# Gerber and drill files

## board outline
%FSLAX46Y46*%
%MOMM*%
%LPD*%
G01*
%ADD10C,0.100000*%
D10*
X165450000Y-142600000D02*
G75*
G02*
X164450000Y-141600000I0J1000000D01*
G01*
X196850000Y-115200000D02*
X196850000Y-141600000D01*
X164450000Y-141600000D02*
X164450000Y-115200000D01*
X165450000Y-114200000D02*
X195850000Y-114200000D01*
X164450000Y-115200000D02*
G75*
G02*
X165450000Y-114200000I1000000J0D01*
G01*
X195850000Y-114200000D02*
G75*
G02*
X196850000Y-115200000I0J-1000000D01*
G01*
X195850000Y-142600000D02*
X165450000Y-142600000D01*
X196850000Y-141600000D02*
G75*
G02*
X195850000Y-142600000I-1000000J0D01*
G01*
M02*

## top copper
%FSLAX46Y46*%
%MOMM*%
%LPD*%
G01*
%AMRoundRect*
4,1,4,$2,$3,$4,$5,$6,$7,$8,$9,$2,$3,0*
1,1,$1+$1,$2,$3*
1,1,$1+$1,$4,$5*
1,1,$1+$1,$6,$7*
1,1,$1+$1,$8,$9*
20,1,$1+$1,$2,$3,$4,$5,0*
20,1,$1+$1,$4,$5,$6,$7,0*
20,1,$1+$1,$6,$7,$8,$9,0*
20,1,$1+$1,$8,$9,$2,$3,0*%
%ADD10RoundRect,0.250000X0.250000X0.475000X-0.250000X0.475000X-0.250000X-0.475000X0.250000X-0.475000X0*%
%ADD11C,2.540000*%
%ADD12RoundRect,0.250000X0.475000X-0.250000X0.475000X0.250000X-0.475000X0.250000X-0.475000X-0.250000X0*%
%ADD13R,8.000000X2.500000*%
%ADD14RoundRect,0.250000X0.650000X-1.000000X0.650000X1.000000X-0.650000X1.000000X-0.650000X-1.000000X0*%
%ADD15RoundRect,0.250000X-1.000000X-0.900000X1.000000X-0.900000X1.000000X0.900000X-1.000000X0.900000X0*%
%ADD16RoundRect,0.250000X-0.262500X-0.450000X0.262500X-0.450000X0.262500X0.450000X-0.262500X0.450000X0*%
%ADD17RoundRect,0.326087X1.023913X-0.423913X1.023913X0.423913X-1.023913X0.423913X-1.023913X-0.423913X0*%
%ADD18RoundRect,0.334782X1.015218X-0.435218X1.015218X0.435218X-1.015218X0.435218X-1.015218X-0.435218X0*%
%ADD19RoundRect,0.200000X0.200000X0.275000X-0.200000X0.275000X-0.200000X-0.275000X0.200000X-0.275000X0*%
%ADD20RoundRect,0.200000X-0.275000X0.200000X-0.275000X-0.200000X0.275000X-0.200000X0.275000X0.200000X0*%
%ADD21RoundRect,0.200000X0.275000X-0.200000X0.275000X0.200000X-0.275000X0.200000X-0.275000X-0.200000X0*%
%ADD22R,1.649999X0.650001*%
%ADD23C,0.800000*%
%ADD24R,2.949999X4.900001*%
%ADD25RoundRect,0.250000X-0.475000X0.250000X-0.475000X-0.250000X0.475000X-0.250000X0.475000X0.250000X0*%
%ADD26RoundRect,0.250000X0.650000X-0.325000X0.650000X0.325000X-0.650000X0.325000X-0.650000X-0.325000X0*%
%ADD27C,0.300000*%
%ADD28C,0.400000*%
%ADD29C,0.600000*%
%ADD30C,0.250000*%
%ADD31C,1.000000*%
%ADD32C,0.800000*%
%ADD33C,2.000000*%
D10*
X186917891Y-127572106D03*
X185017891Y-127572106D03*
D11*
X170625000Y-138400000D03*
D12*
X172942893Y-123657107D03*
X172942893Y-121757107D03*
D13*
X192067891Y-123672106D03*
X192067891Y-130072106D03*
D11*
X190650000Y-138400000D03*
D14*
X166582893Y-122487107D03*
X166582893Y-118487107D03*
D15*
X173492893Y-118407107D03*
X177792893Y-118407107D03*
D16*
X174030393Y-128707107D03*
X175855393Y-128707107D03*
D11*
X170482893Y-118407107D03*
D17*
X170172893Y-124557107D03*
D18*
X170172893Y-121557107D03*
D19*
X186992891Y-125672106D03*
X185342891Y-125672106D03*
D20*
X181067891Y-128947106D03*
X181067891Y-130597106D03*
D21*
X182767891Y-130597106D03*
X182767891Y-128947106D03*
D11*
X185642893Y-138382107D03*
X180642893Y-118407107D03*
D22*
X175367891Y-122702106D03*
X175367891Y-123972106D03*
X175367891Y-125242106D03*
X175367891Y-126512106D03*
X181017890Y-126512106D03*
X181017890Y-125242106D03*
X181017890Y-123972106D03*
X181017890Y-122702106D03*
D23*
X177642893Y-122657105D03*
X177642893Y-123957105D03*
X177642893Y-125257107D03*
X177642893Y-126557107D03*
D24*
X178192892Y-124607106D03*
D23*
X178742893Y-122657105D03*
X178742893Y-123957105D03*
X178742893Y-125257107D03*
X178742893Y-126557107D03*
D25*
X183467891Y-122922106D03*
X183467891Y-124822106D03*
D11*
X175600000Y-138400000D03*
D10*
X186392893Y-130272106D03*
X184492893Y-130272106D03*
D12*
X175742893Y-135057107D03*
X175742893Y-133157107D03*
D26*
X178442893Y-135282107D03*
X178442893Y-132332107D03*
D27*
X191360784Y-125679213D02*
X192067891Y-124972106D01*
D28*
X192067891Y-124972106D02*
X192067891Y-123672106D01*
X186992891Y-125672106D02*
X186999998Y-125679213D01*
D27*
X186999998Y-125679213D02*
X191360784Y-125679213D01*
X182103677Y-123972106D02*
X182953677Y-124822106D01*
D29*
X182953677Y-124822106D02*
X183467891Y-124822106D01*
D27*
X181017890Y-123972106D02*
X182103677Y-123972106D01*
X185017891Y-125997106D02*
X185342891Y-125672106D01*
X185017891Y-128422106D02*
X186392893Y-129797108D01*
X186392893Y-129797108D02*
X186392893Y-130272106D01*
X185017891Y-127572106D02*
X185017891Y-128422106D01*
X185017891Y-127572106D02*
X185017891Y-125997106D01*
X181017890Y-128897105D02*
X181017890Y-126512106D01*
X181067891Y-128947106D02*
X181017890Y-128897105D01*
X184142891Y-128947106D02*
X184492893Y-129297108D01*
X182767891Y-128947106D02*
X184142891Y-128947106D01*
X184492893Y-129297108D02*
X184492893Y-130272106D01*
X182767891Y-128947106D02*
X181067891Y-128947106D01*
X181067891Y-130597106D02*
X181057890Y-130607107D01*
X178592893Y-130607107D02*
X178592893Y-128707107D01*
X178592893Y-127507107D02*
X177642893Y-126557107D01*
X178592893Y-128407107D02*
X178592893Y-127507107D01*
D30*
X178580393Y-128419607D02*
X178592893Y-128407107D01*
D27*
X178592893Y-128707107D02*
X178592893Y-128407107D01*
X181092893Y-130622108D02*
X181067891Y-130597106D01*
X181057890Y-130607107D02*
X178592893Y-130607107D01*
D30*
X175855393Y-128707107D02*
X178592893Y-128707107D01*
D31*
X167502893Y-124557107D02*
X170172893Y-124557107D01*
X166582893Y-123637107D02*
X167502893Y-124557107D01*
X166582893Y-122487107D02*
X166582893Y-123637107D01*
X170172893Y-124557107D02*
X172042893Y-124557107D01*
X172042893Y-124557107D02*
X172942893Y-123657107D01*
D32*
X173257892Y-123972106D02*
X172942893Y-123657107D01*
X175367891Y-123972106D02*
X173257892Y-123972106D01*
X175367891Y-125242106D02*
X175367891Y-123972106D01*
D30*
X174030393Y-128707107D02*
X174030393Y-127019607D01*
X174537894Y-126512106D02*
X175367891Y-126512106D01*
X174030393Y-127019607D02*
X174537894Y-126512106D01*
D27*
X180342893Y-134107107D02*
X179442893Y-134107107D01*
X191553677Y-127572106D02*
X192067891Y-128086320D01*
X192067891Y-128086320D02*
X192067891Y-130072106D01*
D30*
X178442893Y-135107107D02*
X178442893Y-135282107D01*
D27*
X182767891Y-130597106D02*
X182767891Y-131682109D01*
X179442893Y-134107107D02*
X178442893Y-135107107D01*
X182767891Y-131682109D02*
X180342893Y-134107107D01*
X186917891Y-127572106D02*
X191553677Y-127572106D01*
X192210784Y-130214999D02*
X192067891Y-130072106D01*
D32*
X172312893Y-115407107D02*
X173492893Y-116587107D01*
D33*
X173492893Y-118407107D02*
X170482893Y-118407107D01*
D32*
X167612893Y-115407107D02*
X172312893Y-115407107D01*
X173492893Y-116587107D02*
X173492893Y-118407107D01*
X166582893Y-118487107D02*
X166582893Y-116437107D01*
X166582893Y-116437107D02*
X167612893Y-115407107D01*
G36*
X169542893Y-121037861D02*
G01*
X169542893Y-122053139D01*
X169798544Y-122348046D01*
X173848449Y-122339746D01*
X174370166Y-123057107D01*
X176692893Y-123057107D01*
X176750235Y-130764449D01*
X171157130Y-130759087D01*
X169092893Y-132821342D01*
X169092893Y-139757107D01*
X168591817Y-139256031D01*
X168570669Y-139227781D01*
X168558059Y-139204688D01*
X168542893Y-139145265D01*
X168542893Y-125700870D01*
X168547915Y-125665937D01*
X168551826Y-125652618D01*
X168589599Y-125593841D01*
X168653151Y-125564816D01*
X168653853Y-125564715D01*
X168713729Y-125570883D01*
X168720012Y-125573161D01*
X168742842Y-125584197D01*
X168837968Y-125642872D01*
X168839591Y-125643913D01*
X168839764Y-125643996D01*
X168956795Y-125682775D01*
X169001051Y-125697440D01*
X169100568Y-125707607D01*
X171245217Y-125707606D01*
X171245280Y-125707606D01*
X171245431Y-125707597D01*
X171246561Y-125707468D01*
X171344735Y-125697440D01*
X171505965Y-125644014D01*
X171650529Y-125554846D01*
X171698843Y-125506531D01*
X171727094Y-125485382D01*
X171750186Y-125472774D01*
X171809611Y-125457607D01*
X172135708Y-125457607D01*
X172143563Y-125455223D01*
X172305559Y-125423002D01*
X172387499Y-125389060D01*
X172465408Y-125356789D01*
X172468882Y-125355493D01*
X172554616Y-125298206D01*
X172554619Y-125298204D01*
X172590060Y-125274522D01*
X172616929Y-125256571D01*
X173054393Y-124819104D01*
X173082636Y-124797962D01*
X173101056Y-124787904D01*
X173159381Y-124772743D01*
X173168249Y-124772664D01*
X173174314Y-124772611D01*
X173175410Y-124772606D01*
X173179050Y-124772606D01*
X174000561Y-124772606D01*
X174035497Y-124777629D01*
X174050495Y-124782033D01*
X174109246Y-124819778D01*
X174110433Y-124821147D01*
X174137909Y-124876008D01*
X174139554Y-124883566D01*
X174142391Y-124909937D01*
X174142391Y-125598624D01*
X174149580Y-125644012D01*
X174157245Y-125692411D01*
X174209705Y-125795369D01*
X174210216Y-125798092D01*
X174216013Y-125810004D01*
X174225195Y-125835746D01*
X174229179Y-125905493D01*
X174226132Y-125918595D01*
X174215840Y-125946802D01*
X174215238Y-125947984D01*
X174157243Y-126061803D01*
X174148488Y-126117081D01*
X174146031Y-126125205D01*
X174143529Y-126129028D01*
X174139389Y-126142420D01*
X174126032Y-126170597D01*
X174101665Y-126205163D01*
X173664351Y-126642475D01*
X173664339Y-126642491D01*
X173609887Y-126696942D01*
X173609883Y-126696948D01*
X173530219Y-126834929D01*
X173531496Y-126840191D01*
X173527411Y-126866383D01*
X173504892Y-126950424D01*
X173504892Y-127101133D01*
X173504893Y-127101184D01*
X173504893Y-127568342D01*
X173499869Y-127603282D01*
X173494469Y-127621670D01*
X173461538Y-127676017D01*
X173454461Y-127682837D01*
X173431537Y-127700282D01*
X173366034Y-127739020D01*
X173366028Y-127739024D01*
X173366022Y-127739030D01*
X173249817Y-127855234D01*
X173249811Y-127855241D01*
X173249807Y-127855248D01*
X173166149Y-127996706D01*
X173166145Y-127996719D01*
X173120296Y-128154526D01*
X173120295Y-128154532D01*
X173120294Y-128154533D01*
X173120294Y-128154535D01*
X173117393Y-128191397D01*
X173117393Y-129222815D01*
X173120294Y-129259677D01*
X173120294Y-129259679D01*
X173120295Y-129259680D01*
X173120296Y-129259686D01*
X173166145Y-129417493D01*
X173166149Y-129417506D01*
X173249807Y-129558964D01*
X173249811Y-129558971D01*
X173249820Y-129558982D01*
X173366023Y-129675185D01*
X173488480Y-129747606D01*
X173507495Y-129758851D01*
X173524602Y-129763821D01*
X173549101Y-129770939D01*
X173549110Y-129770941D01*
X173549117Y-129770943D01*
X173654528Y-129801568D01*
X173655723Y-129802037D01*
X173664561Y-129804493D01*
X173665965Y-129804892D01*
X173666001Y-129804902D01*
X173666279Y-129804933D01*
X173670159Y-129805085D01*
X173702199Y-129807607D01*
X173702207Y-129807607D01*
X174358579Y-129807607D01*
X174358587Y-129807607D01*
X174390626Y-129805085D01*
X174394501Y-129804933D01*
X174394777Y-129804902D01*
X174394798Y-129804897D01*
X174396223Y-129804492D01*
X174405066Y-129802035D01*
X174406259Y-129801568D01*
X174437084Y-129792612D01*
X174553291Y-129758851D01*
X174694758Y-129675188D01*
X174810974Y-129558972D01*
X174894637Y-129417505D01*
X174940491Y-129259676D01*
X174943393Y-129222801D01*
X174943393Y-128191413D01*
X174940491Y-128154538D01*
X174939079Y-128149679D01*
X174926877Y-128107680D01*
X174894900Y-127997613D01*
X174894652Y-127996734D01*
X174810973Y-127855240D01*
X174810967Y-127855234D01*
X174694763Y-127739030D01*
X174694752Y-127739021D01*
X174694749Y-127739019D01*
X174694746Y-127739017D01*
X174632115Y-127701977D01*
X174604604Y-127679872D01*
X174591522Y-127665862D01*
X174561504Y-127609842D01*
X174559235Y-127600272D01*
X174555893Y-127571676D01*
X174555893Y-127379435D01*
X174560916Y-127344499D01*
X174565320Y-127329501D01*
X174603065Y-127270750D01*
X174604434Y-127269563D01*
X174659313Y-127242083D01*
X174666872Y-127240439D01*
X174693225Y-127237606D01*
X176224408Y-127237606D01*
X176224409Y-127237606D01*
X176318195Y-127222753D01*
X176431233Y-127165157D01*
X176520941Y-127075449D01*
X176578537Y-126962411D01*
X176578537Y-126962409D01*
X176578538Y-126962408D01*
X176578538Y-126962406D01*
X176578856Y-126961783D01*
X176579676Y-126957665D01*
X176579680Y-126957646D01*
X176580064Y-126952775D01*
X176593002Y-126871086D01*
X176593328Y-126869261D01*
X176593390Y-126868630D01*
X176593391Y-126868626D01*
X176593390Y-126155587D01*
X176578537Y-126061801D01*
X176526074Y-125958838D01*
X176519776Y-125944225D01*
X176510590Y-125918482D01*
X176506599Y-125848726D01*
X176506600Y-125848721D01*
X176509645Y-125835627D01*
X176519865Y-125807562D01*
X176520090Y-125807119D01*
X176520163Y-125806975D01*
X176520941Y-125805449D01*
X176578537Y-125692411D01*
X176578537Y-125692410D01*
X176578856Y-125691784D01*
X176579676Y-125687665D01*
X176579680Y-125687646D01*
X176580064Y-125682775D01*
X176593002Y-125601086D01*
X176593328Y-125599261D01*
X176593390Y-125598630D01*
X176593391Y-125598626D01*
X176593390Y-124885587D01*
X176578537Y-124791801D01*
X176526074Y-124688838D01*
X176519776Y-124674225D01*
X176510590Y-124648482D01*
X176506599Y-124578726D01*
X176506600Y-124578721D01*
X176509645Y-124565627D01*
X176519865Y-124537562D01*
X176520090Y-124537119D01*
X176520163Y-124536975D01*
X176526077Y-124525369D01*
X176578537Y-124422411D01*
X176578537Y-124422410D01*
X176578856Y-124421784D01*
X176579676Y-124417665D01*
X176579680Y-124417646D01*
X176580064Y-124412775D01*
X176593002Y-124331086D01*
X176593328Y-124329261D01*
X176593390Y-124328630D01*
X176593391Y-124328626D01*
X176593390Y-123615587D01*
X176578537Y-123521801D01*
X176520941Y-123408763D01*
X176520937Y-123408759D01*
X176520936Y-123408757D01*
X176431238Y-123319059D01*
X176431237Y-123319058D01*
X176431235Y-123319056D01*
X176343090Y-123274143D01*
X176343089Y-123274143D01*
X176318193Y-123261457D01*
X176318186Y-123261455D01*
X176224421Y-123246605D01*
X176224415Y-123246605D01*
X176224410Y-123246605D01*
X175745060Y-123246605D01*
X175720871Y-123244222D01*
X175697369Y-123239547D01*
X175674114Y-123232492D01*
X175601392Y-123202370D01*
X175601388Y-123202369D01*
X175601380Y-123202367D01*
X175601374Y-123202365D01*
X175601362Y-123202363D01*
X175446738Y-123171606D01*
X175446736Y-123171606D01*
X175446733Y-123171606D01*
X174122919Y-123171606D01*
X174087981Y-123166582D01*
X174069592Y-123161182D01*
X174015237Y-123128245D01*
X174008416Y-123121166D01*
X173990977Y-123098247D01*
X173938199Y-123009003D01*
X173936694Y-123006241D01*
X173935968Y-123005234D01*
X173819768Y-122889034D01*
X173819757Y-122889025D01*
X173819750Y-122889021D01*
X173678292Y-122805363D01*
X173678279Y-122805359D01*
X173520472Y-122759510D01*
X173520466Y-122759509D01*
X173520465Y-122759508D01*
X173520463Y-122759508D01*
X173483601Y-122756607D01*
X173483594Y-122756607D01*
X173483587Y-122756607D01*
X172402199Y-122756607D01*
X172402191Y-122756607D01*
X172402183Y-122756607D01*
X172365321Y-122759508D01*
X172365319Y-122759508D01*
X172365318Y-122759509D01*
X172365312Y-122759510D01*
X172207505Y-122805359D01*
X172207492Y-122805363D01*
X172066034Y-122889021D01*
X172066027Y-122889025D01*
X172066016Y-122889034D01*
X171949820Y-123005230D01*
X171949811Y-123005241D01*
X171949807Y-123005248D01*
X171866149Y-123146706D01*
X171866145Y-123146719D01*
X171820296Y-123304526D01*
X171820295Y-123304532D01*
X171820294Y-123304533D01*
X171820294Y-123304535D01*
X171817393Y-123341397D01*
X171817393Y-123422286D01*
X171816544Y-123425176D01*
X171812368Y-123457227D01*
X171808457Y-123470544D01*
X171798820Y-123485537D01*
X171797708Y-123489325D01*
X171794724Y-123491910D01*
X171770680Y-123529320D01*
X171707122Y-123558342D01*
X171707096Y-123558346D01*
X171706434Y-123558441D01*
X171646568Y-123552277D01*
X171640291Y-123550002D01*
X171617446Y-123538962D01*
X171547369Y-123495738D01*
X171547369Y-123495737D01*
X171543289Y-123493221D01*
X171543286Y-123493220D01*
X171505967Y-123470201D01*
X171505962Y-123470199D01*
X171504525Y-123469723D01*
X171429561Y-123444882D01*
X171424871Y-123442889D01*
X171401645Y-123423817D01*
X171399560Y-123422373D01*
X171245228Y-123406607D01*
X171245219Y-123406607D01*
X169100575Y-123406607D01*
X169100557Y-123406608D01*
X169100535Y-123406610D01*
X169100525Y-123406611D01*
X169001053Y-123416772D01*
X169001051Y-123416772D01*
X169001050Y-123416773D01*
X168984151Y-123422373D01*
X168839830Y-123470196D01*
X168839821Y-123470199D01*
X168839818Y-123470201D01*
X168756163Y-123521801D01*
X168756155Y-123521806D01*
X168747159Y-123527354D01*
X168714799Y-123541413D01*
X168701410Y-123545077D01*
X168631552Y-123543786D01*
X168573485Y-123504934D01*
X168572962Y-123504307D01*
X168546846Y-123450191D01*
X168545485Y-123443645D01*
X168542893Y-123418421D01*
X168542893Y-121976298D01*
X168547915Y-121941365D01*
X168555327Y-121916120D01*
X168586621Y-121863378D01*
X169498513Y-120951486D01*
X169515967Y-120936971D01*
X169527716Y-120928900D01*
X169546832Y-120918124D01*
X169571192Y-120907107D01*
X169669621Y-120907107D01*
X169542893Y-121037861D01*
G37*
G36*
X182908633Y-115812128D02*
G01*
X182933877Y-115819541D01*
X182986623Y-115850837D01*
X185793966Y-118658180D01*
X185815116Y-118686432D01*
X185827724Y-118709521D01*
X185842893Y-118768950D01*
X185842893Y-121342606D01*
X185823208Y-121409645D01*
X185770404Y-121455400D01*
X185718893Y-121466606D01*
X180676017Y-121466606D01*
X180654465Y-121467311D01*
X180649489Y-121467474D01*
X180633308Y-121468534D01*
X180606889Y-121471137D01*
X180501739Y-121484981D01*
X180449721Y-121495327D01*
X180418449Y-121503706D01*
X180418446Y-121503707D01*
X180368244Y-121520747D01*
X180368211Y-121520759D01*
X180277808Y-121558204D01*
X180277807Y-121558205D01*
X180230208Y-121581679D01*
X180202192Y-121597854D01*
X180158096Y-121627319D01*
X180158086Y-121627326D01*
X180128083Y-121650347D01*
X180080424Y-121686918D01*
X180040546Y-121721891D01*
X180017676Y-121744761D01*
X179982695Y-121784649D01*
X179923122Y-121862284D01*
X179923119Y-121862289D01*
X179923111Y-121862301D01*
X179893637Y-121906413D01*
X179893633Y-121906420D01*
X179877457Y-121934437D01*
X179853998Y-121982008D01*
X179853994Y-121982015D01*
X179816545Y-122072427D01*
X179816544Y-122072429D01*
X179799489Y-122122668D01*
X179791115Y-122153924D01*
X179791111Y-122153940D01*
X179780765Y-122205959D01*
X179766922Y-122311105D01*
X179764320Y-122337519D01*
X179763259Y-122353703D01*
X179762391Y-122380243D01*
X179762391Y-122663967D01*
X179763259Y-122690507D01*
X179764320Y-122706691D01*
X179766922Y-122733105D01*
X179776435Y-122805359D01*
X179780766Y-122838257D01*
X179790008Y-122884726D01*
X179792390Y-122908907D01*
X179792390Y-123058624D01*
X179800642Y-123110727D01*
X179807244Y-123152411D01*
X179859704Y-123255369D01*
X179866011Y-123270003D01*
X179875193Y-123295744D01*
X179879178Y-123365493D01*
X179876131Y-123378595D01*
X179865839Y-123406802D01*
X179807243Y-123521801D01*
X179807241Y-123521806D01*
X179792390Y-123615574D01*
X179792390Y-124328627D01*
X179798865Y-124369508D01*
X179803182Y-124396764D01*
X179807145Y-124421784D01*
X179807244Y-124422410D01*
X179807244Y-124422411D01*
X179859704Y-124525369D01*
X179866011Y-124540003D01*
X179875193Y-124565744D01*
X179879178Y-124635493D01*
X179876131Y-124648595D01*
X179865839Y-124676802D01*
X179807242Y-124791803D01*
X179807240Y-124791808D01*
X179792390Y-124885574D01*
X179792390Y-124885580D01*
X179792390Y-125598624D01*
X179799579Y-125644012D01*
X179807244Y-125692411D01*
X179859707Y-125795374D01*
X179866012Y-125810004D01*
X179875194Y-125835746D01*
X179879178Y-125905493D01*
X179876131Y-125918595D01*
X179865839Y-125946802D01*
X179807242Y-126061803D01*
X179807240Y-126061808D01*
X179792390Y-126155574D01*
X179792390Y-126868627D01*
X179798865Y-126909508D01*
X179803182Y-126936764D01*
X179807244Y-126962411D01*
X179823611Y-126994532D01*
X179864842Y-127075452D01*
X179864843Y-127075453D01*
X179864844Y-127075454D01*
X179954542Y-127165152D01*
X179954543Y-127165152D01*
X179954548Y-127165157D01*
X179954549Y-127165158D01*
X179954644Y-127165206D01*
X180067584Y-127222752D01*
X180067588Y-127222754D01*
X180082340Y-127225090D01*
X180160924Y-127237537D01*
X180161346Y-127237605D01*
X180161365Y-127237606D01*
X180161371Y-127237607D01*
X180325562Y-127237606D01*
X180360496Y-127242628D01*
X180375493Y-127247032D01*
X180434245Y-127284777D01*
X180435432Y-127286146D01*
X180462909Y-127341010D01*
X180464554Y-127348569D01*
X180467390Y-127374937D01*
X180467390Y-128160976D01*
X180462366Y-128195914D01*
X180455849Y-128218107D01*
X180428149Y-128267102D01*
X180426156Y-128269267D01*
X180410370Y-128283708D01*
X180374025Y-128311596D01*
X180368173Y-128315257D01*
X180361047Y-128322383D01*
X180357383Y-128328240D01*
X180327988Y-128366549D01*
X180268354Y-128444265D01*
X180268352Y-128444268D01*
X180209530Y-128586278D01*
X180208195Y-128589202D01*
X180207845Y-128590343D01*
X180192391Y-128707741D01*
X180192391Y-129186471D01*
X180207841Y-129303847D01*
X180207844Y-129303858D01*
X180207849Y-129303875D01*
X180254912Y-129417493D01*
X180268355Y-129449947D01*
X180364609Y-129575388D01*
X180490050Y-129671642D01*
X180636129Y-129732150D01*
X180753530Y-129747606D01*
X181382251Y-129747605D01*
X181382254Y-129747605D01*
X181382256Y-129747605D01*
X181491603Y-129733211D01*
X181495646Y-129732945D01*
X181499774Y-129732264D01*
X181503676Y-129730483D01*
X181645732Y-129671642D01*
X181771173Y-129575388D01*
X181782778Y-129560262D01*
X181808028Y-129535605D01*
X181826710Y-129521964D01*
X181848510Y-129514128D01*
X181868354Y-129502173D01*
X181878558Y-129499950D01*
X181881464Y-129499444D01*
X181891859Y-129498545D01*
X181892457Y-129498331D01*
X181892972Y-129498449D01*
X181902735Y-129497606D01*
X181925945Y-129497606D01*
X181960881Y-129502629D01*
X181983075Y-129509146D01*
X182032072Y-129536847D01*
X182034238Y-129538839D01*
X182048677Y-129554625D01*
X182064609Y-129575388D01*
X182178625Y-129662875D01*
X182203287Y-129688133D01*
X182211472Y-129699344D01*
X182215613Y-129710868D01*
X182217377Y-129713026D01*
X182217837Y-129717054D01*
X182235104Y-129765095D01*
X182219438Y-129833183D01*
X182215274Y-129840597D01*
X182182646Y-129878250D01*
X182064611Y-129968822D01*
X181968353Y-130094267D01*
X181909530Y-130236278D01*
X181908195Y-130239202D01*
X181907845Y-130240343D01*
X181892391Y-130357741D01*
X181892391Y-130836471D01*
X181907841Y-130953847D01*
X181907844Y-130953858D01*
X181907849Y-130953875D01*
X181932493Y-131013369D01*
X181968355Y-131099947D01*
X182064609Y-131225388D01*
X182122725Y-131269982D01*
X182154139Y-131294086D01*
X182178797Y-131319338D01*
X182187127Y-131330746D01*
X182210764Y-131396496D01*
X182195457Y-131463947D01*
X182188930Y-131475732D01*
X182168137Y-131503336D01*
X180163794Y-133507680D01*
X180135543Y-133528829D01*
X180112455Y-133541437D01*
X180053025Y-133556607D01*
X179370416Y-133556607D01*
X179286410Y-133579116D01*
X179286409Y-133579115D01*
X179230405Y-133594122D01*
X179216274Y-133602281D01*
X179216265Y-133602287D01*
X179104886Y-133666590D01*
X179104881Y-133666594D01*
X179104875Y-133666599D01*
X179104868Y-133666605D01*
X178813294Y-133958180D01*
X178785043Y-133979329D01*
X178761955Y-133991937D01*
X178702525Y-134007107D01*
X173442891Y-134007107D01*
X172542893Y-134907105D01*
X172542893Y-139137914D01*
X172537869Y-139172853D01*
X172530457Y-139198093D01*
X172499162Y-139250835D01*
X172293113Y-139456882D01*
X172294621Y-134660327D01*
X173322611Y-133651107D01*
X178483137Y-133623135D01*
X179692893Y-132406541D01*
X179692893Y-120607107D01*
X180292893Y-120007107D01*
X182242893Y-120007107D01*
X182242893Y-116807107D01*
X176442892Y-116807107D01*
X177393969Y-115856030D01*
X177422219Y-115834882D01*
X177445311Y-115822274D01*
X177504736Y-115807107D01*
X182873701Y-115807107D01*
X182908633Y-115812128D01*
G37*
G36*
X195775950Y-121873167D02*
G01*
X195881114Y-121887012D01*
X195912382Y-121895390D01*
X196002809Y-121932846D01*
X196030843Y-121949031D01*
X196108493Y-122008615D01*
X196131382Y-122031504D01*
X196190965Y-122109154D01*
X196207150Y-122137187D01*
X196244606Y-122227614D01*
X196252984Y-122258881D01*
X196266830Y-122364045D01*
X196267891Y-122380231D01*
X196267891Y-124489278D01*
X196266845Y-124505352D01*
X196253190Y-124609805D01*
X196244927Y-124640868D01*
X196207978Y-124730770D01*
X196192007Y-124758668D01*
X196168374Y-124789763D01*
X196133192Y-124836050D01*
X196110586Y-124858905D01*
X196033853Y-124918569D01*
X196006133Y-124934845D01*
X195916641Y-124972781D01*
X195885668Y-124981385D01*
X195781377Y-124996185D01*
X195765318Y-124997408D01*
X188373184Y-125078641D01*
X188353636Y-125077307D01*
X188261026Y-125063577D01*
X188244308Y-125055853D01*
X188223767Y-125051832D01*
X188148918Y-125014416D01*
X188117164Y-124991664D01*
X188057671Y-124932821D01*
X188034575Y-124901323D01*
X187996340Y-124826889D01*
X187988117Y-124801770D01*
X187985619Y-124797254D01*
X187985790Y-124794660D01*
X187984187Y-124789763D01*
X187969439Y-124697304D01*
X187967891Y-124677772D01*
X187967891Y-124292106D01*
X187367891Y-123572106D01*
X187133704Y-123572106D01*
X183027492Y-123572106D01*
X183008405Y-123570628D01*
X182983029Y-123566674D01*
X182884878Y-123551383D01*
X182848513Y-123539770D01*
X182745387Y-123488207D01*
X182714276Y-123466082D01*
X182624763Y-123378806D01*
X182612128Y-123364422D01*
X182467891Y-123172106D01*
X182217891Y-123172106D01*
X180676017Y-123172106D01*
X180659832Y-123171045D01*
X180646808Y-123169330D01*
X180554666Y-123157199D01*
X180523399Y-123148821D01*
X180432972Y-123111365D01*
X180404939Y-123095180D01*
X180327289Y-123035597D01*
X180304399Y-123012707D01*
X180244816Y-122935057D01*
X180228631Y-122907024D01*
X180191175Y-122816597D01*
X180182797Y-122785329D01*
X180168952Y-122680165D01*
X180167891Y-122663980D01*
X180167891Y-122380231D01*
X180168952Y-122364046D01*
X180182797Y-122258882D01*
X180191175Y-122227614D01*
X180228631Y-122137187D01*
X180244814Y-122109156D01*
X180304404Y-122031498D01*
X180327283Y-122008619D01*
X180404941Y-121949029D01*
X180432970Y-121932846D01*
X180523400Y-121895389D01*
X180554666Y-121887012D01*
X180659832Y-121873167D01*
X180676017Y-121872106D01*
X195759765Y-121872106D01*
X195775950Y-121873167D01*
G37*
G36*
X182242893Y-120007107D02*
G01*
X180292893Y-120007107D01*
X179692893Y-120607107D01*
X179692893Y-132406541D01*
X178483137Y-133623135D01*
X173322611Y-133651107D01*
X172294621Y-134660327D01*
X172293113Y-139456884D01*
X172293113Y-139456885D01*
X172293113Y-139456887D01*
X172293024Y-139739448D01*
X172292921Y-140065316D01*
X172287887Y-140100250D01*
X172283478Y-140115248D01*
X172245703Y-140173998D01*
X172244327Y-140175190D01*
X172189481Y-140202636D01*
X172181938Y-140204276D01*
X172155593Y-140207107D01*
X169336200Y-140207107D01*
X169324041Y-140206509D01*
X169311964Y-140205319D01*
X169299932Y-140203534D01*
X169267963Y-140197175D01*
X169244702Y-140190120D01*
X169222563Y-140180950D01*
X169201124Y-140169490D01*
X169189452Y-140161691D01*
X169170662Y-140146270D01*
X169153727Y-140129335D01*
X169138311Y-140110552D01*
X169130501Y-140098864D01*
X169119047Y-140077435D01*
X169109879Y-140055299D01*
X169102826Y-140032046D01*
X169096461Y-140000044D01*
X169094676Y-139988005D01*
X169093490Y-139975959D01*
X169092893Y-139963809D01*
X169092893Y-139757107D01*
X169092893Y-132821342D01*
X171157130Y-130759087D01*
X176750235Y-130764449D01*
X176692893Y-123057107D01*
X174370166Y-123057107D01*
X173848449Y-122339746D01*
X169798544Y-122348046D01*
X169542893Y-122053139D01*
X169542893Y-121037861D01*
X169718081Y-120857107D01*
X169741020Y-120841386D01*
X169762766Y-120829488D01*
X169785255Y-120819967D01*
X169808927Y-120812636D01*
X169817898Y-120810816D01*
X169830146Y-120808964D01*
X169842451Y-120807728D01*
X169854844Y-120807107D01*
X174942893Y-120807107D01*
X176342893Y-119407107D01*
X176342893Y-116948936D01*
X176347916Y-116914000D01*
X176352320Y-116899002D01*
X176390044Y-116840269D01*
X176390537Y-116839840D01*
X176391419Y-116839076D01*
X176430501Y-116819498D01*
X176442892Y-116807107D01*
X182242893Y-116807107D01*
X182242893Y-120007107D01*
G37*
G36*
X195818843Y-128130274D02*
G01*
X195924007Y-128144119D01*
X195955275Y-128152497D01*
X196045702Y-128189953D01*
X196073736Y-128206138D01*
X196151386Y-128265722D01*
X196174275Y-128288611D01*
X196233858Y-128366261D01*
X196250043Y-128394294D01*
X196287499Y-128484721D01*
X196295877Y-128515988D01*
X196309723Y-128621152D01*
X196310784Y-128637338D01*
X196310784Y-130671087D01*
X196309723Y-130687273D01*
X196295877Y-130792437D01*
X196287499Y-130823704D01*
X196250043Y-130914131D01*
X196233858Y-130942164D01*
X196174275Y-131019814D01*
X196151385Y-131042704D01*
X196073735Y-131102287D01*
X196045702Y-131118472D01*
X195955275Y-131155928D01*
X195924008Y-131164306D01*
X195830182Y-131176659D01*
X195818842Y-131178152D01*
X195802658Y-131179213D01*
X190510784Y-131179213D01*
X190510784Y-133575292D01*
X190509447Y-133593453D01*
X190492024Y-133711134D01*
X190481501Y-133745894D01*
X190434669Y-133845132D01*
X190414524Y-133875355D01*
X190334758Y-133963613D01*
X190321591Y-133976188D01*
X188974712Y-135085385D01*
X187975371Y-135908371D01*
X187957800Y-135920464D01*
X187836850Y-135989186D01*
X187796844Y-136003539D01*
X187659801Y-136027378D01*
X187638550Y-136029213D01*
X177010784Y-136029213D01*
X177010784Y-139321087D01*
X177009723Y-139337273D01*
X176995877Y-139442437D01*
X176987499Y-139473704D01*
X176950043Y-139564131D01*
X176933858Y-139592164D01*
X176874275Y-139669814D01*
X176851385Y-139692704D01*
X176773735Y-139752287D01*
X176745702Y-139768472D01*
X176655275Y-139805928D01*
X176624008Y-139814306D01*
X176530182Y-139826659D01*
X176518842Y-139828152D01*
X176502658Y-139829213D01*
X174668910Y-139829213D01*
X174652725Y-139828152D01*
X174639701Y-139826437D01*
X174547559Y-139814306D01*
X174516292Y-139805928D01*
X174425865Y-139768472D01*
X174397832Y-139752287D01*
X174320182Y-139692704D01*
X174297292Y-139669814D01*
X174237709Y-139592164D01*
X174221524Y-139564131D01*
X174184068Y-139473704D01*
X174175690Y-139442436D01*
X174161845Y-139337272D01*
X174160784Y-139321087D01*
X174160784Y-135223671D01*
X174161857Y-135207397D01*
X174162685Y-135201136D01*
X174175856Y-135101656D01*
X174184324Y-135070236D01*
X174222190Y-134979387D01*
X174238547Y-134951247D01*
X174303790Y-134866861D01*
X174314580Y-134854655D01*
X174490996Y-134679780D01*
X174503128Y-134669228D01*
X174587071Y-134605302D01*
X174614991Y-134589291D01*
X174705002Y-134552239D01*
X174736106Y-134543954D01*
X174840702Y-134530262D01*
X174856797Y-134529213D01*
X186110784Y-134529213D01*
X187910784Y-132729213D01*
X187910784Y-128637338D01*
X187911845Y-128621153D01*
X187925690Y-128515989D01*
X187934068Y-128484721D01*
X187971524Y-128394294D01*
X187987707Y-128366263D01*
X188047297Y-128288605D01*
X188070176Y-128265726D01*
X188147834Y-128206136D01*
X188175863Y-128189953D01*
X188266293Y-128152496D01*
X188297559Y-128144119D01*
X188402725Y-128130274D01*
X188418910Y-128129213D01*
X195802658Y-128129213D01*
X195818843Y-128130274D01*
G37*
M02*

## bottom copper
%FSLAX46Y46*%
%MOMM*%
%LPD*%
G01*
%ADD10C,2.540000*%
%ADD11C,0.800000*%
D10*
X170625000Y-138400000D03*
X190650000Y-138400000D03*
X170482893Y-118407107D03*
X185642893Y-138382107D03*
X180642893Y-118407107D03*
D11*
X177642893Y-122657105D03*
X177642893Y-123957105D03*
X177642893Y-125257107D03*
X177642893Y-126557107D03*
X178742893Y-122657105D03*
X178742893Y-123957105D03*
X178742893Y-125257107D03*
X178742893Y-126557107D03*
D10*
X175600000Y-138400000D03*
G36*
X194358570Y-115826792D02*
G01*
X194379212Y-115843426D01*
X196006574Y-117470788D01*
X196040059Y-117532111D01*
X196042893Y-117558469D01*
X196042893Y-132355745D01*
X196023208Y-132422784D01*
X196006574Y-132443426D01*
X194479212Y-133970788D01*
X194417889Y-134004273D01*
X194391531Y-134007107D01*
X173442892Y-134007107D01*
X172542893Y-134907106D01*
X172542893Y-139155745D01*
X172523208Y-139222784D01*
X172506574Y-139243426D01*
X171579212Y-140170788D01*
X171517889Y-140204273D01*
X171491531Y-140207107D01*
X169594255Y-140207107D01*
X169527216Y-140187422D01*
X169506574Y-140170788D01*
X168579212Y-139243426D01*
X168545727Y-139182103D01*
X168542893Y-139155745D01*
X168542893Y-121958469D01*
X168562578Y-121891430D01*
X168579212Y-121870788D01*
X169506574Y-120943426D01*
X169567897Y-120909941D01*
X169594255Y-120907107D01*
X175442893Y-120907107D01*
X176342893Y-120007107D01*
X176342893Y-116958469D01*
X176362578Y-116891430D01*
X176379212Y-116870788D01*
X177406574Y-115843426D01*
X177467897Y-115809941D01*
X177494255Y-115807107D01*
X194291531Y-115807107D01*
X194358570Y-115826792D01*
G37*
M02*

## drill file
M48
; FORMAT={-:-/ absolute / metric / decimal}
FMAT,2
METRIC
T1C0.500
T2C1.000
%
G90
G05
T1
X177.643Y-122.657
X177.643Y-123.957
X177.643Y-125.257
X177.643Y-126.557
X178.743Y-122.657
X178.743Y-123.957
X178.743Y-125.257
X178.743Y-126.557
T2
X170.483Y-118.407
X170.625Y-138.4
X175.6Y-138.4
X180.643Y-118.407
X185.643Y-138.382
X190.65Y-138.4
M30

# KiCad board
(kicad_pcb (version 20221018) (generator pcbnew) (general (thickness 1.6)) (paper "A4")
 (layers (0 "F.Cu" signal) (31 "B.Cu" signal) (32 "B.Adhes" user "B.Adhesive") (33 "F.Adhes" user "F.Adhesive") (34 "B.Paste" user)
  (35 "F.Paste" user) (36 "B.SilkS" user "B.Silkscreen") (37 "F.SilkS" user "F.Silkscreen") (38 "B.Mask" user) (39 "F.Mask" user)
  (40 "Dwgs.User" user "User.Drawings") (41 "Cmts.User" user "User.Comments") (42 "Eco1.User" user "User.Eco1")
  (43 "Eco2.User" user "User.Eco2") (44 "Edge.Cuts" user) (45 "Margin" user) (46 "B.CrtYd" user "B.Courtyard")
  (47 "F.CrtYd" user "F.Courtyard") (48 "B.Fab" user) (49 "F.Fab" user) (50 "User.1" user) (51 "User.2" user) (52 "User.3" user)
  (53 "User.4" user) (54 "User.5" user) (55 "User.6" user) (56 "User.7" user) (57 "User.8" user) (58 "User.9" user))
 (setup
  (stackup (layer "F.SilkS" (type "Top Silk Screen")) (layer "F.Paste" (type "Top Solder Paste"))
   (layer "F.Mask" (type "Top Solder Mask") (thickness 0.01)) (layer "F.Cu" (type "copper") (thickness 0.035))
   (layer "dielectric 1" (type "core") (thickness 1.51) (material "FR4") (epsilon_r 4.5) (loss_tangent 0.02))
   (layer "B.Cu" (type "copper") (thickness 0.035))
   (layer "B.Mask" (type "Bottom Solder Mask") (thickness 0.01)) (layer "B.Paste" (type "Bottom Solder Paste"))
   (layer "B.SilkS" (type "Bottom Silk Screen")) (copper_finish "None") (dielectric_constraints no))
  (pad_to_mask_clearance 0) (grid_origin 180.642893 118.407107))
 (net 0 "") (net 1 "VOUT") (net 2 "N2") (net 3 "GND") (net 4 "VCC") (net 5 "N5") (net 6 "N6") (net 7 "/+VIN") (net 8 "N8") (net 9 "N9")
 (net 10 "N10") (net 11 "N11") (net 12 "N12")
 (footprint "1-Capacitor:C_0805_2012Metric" (layer "F.Cu") (at 185.967891 127.572106 180)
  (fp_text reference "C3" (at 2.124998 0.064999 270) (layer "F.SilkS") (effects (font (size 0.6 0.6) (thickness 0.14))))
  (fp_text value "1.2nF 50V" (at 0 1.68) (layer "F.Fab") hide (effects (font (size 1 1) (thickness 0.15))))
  (pad "1" smd roundrect (at -0.95 0 180) (size 1 1.45) (layers "F.Cu" "F.Paste" "F.Mask") (roundrect_rratio 0.25) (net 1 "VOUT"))
  (pad "2" smd roundrect (at 0.95 0 180) (size 1 1.45) (layers "F.Cu" "F.Paste" "F.Mask") (roundrect_rratio 0.25) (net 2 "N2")))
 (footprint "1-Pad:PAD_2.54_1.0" (layer "F.Cu") (at 170.625 138.4)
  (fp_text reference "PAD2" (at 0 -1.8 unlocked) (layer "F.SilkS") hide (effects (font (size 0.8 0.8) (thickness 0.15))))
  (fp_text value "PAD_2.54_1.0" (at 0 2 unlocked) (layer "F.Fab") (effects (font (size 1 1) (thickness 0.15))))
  (pad "1" thru_hole circle (at 0 0) (size 2.54 2.54) (drill 1) (layers "*.Cu" "*.Mask") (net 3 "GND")))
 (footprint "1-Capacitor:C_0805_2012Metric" (layer "F.Cu") (at 172.942893 122.707107 90)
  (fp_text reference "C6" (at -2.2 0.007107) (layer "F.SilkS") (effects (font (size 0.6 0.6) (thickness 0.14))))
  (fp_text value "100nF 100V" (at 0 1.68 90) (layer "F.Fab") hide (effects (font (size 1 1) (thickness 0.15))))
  (pad "1" smd roundrect (at -0.95 0 90) (size 1 1.45) (layers "F.Cu" "F.Paste" "F.Mask") (roundrect_rratio 0.25) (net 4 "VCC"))
  (pad "2" smd roundrect (at 0.95 0 90) (size 1 1.45) (layers "F.Cu" "F.Paste" "F.Mask") (roundrect_rratio 0.25) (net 3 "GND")))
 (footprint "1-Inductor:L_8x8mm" (layer "F.Cu") (at 192.067891 126.872106 -90)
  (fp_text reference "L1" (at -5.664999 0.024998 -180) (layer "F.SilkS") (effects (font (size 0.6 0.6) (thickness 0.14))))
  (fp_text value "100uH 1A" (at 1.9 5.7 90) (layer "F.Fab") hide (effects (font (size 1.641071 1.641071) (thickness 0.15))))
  (pad "1" smd rect (at -3.2 0) (size 8 2.5) (layers "F.Cu" "F.Paste" "F.Mask") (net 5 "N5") (solder_mask_margin 0.102))
  (pad "2" smd rect (at 3.2 0) (size 8 2.5) (layers "F.Cu" "F.Paste" "F.Mask") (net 1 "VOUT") (solder_mask_margin 0.102)))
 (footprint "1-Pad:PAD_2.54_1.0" (layer "F.Cu") (at 190.65 138.4)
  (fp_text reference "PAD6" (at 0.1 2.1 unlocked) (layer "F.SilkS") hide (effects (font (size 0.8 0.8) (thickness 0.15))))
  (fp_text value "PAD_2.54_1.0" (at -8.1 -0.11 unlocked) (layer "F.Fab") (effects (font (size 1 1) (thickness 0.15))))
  (pad "1" thru_hole circle (at 0 0) (size 2.54 2.54) (drill 1) (layers "*.Cu" "*.Mask") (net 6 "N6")))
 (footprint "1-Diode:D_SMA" (layer "F.Cu") (at 166.582893 120.487107 90)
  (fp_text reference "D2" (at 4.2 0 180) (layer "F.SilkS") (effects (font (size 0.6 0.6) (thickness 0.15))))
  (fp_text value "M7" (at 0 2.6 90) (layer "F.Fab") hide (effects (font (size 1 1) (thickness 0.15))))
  (pad "1" smd roundrect (at -2 0 90) (size 2.5 1.8) (layers "F.Cu" "F.Paste" "F.Mask") (roundrect_rratio 0.1388888889) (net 4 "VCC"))
  (pad "2" smd roundrect (at 2 0 90) (size 2.5 1.8) (layers "F.Cu" "F.Paste" "F.Mask") (roundrect_rratio 0.1388888889) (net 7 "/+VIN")))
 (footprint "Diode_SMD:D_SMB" (layer "F.Cu") (at 175.642893 118.407107)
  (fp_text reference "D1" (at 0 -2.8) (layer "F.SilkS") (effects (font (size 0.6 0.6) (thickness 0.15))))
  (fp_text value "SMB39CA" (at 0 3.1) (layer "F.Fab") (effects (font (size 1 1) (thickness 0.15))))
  (pad "1" smd roundrect (at -2.15 0) (size 2.5 2.3) (layers "F.Cu" "F.Paste" "F.Mask") (roundrect_rratio 0.1086956522) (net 7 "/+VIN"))
  (pad "2" smd roundrect (at 2.15 0) (size 2.5 2.3) (layers "F.Cu" "F.Paste" "F.Mask") (roundrect_rratio 0.1086956522) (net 3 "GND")))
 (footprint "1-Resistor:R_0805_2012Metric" (layer "F.Cu") (at 174.942893 128.707107)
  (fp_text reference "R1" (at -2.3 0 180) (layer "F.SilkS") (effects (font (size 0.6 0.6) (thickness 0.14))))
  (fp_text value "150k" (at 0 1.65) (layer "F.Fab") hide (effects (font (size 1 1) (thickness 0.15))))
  (pad "1" smd roundrect (at -0.9125 0) (size 1.025 1.4) (layers "F.Cu" "F.Paste" "F.Mask") (roundrect_rratio 0.243902439) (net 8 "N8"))
  (pad "2" smd roundrect (at 0.9125 0) (size 1.025 1.4) (layers "F.Cu" "F.Paste" "F.Mask") (roundrect_rratio 0.243902439) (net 3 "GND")))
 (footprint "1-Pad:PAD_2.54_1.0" (layer "F.Cu") (at 172.717893 118.332107)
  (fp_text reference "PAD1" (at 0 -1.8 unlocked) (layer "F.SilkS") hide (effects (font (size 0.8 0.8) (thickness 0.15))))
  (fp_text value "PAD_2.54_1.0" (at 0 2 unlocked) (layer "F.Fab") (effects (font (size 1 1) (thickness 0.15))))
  (pad "1" thru_hole circle (at -2.235 0.075) (size 2.54 2.54) (drill 1) (layers "*.Cu" "*.Mask") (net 7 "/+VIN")))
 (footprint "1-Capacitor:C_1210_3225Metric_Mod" (layer "F.Cu") (at 170.172893 123.057107 90)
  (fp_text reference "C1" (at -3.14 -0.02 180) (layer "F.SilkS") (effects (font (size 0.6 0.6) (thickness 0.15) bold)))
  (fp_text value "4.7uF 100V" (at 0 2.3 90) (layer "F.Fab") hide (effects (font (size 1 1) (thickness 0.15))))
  (pad "1" smd roundrect (at -1.5 0 90) (size 1.5 2.7) (layers "F.Cu" "F.Paste" "F.Mask") (roundrect_rratio 0.2173913333) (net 4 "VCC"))
  (pad "2" smd roundrect (at 1.5 0 90) (size 1.54 2.7) (layers "F.Cu" "F.Paste" "F.Mask") (roundrect_rratio 0.2173909091) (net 3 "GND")))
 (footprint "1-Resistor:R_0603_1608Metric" (layer "F.Cu") (at 186.167891 125.672106 180)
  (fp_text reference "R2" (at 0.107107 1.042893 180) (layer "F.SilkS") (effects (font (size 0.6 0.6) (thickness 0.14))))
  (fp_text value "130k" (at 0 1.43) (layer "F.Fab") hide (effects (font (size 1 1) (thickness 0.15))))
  (pad "1" smd roundrect (at -0.825 0 180) (size 0.8 0.95) (layers "F.Cu" "F.Paste" "F.Mask") (roundrect_rratio 0.25) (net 5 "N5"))
  (pad "2" smd roundrect (at 0.825 0 180) (size 0.8 0.95) (layers "F.Cu" "F.Paste" "F.Mask") (roundrect_rratio 0.25) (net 2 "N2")))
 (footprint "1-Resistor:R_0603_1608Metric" (layer "F.Cu") (at 181.067891 129.772106 -90)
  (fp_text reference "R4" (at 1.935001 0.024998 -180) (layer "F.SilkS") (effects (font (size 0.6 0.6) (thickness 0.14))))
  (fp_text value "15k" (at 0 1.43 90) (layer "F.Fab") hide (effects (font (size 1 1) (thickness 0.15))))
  (pad "1" smd roundrect (at -0.825 0 270) (size 0.8 0.95) (layers "F.Cu" "F.Paste" "F.Mask") (roundrect_rratio 0.25) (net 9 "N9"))
  (pad "2" smd roundrect (at 0.825 0 270) (size 0.8 0.95) (layers "F.Cu" "F.Paste" "F.Mask") (roundrect_rratio 0.25) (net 3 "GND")))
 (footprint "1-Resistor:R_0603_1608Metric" (layer "F.Cu") (at 182.767891 129.772106 90)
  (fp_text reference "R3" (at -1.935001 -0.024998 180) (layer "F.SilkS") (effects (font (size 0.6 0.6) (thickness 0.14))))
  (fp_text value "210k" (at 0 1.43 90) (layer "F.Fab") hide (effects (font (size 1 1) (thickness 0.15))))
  (pad "1" smd roundrect (at -0.825 0 90) (size 0.8 0.95) (layers "F.Cu" "F.Paste" "F.Mask") (roundrect_rratio 0.25) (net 1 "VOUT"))
  (pad "2" smd roundrect (at 0.825 0 90) (size 0.8 0.95) (layers "F.Cu" "F.Paste" "F.Mask") (roundrect_rratio 0.25) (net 9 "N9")))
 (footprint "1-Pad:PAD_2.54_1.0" (layer "F.Cu") (at 185.642893 138.382107)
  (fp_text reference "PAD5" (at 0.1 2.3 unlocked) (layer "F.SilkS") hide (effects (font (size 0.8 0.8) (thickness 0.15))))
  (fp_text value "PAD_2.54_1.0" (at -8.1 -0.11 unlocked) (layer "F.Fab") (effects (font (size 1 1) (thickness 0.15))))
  (pad "1" thru_hole circle (at 0 0) (size 2.54 2.54) (drill 1) (layers "*.Cu" "*.Mask") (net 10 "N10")))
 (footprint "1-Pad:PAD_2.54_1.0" (layer "F.Cu") (at 180.642893 118.407107)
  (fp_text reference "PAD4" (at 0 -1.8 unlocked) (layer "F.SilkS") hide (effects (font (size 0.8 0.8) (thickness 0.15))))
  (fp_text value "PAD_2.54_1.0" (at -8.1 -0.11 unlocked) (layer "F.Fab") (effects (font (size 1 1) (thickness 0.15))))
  (pad "1" thru_hole circle (at 0 0) (size 2.54 2.54) (drill 1) (layers "*.Cu" "*.Mask") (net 3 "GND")))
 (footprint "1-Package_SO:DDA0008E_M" (layer "F.Cu") (at 178.192892 124.607106)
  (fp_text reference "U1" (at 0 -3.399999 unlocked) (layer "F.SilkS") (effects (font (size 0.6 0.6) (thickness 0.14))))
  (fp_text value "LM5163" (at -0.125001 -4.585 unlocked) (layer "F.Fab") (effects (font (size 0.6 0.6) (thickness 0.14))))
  (pad "1" smd rect (at -2.825001 -1.905 90) (size 0.650001 1.649999) (layers "F.Cu" "F.Paste" "F.Mask") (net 3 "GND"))
  (pad "2" smd rect (at -2.825001 -0.635 90) (size 0.650001 1.649999) (layers "F.Cu" "F.Paste" "F.Mask") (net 4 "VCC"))
  (pad "3" smd rect (at -2.825001 0.635 90) (size 0.650001 1.649999) (layers "F.Cu" "F.Paste" "F.Mask") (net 4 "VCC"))
  (pad "4" smd rect (at -2.825001 1.905 90) (size 0.650001 1.649999) (layers "F.Cu" "F.Paste" "F.Mask") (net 8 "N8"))
  (pad "5" smd rect (at 2.824998 1.905 90) (size 0.650001 1.649999) (layers "F.Cu" "F.Paste" "F.Mask") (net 9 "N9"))
  (pad "6" smd rect (at 2.824998 0.635 90) (size 0.650001 1.649999) (layers "F.Cu" "F.Paste" "F.Mask") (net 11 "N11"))
  (pad "7" smd rect (at 2.824998 -0.635 90) (size 0.650001 1.649999) (layers "F.Cu" "F.Paste" "F.Mask") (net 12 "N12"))
  (pad "8" smd rect (at 2.824998 -1.905 90) (size 0.650001 1.649999) (layers "F.Cu" "F.Paste" "F.Mask") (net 5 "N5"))
  (pad "9" thru_hole circle (at -0.549999 -1.950001) (size 0.8 0.8) (drill 0.5) (layers "*.Cu" "*.Mask") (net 3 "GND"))
  (pad "9" thru_hole circle (at -0.549999 -0.650001) (size 0.8 0.8) (drill 0.5) (layers "*.Cu" "*.Mask") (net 3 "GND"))
  (pad "9" thru_hole circle (at -0.549999 0.650001) (size 0.8 0.8) (drill 0.5) (layers "*.Cu" "*.Mask") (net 3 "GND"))
  (pad "9" thru_hole circle (at -0.549999 1.950001) (size 0.8 0.8) (drill 0.5) (layers "*.Cu" "*.Mask") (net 3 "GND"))
  (pad "9" smd rect (at 0 0) (size 2.949999 4.900001) (layers "F.Cu") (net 3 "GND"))
  (pad "9" thru_hole circle (at 0.550001 -1.950001) (size 0.8 0.8) (drill 0.5) (layers "*.Cu" "*.Mask") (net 3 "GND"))
  (pad "9" thru_hole circle (at 0.550001 -0.650001) (size 0.8 0.8) (drill 0.5) (layers "*.Cu" "*.Mask") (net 3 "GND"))
  (pad "9" thru_hole circle (at 0.550001 0.650001) (size 0.8 0.8) (drill 0.5) (layers "*.Cu" "*.Mask") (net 3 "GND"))
  (pad "9" thru_hole circle (at 0.550001 1.950001) (size 0.8 0.8) (drill 0.5) (layers "*.Cu" "*.Mask") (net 3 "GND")))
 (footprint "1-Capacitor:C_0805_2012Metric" (layer "F.Cu") (at 183.467891 123.872106 -90)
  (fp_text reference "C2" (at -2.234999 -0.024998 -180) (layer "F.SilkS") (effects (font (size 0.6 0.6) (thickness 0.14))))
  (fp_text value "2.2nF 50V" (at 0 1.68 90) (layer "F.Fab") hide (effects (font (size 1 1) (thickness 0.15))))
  (pad "1" smd roundrect (at -0.95 0 270) (size 1 1.45) (layers "F.Cu" "F.Paste" "F.Mask") (roundrect_rratio 0.25) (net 5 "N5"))
  (pad "2" smd roundrect (at 0.95 0 270) (size 1 1.45) (layers "F.Cu" "F.Paste" "F.Mask") (roundrect_rratio 0.25) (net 12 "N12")))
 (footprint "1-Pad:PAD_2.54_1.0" (layer "F.Cu") (at 175.6 138.4)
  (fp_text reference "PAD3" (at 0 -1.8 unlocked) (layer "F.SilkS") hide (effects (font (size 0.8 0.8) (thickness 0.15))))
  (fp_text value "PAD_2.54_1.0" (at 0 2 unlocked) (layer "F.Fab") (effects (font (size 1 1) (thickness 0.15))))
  (pad "1" thru_hole circle (at 0 0) (size 2.54 2.54) (drill 1) (layers "*.Cu" "*.Mask") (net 1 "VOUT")))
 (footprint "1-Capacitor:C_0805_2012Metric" (layer "F.Cu") (at 185.442893 130.272106 180)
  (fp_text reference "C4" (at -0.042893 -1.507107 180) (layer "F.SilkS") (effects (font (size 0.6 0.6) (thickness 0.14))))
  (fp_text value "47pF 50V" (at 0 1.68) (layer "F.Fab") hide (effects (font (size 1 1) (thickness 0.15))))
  (pad "1" smd roundrect (at -0.95 0 180) (size 1 1.45) (layers "F.Cu" "F.Paste" "F.Mask") (roundrect_rratio 0.25) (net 2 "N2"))
  (pad "2" smd roundrect (at 0.95 0 180) (size 1 1.45) (layers "F.Cu" "F.Paste" "F.Mask") (roundrect_rratio 0.25) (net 9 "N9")))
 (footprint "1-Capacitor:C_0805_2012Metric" (layer "F.Cu") (at 175.742893 134.107107 90)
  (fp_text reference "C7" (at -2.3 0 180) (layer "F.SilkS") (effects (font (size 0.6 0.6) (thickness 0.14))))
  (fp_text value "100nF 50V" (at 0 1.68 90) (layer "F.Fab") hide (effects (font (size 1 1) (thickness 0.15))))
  (pad "1" smd roundrect (at -0.95 0 90) (size 1 1.45) (layers "F.Cu" "F.Paste" "F.Mask") (roundrect_rratio 0.25) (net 1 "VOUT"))
  (pad "2" smd roundrect (at 0.95 0 90) (size 1 1.45) (layers "F.Cu" "F.Paste" "F.Mask") (roundrect_rratio 0.25) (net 3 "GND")))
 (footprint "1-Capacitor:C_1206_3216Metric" (layer "F.Cu") (at 178.442893 133.807107 90)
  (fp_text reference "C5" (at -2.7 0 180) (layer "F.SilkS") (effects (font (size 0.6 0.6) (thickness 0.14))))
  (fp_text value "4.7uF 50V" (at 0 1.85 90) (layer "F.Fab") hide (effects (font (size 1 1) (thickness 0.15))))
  (pad "1" smd roundrect (at -1.475 0 90) (size 1.15 1.8) (layers "F.Cu" "F.Paste" "F.Mask") (roundrect_rratio 0.2173913043) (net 1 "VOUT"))
  (pad "2" smd roundrect (at 1.475 0 90) (size 1.15 1.8) (layers "F.Cu" "F.Paste" "F.Mask") (roundrect_rratio 0.2173913043) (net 3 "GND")))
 (gr_arc (start 165.45 142.6) (mid 164.742891 142.307109) (end 164.45 141.6) (stroke (width 0.1) (type default)) (layer "Edge.Cuts"))
 (gr_line (start 196.85 115.2) (end 196.85 141.6) (stroke (width 0.1) (type default)) (layer "Edge.Cuts"))
 (gr_line (start 164.45 141.6) (end 164.45 115.2) (stroke (width 0.1) (type default)) (layer "Edge.Cuts"))
 (gr_line (start 165.45 114.2) (end 195.85 114.2) (stroke (width 0.1) (type default)) (layer "Edge.Cuts"))
 (gr_arc (start 164.45 115.2) (mid 164.742898 114.492898) (end 165.45 114.2) (stroke (width 0.1) (type default)) (layer "Edge.Cuts"))
 (gr_arc (start 195.85 114.2) (mid 196.557105 114.492895) (end 196.85 115.2) (stroke (width 0.1) (type default)) (layer "Edge.Cuts"))
 (gr_line (start 195.85 142.6) (end 165.45 142.6) (stroke (width 0.1) (type default)) (layer "Edge.Cuts"))
 (gr_arc (start 196.85 141.6) (mid 196.557112 142.307112) (end 195.85 142.6) (stroke (width 0.1) (type default)) (layer "Edge.Cuts"))
 (segment (start 191.360784 125.679213) (end 192.067891 124.972106) (width 0.3) (layer "F.Cu") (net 5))
 (segment (start 192.067891 124.972106) (end 192.067891 123.672106) (width 0.4) (layer "F.Cu") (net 5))
 (segment (start 186.992891 125.672106) (end 186.999998 125.679213) (width 0.4) (layer "F.Cu") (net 5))
 (segment (start 186.999998 125.679213) (end 191.360784 125.679213) (width 0.3) (layer "F.Cu") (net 5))
 (segment (start 182.103677 123.972106) (end 182.953677 124.822106) (width 0.3) (layer "F.Cu") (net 12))
 (segment (start 182.953677 124.822106) (end 183.467891 124.822106) (width 0.6) (layer "F.Cu") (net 12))
 (segment (start 181.01789 123.972106) (end 182.103677 123.972106) (width 0.3) (layer "F.Cu") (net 12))
 (segment (start 185.017891 125.997106) (end 185.342891 125.672106) (width 0.3) (layer "F.Cu") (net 2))
 (segment (start 185.017891 128.422106) (end 186.392893 129.797108) (width 0.3) (layer "F.Cu") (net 2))
 (segment (start 186.392893 129.797108) (end 186.392893 130.272106) (width 0.3) (layer "F.Cu") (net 2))
 (segment (start 185.017891 127.572106) (end 185.017891 128.422106) (width 0.3) (layer "F.Cu") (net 2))
 (segment (start 185.017891 127.572106) (end 185.017891 125.997106) (width 0.3) (layer "F.Cu") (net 2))
 (segment (start 181.01789 128.897105) (end 181.01789 126.512106) (width 0.3) (layer "F.Cu") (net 9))
 (segment (start 181.067891 128.947106) (end 181.01789 128.897105) (width 0.3) (layer "F.Cu") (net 9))
 (segment (start 184.142891 128.947106) (end 184.492893 129.297108) (width 0.3) (layer "F.Cu") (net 9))
 (segment (start 182.767891 128.947106) (end 184.142891 128.947106) (width 0.3) (layer "F.Cu") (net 9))
 (segment (start 184.492893 129.297108) (end 184.492893 130.272106) (width 0.3) (layer "F.Cu") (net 9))
 (segment (start 182.767891 128.947106) (end 181.067891 128.947106) (width 0.3) (layer "F.Cu") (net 9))
 (segment (start 181.067891 130.597106) (end 181.05789 130.607107) (width 0.3) (layer "F.Cu") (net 3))
 (segment (start 178.592893 130.607107) (end 178.592893 128.707107) (width 0.3) (layer "F.Cu") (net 3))
 (segment (start 178.592893 127.507107) (end 177.642893 126.557107) (width 0.3) (layer "F.Cu") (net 3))
 (segment (start 178.592893 128.407107) (end 178.592893 127.507107) (width 0.3) (layer "F.Cu") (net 3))
 (segment (start 178.580393 128.419607) (end 178.592893 128.407107) (width 0.25) (layer "F.Cu") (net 3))
 (segment (start 178.592893 128.707107) (end 178.592893 128.407107) (width 0.3) (layer "F.Cu") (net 3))
 (segment (start 181.092893 130.622108) (end 181.067891 130.597106) (width 0.3) (layer "F.Cu") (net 3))
 (segment (start 181.05789 130.607107) (end 178.592893 130.607107) (width 0.3) (layer "F.Cu") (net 3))
 (segment (start 175.855393 128.707107) (end 178.592893 128.707107) (width 0.25) (layer "F.Cu") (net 3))
 (segment (start 167.502893 124.557107) (end 170.172893 124.557107) (width 1) (layer "F.Cu") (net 4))
 (segment (start 166.582893 123.637107) (end 167.502893 124.557107) (width 1) (layer "F.Cu") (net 4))
 (segment (start 166.582893 122.487107) (end 166.582893 123.637107) (width 1) (layer "F.Cu") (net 4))
 (segment (start 170.172893 124.557107) (end 172.042893 124.557107) (width 1) (layer "F.Cu") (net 4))
 (segment (start 172.042893 124.557107) (end 172.942893 123.657107) (width 1) (layer "F.Cu") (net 4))
 (segment (start 173.257892 123.972106) (end 172.942893 123.657107) (width 0.8) (layer "F.Cu") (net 4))
 (segment (start 175.367891 123.972106) (end 173.257892 123.972106) (width 0.8) (layer "F.Cu") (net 4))
 (segment (start 175.367891 125.242106) (end 175.367891 123.972106) (width 0.8) (layer "F.Cu") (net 4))
 (segment (start 174.030393 128.707107) (end 174.030393 127.019607) (width 0.25) (layer "F.Cu") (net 8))
 (segment (start 174.537894 126.512106) (end 175.367891 126.512106) (width 0.25) (layer "F.Cu") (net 8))
 (segment (start 174.030393 127.019607) (end 174.537894 126.512106) (width 0.25) (layer "F.Cu") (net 8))
 (segment (start 180.342893 134.107107) (end 179.442893 134.107107) (width 0.3) (layer "F.Cu") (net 1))
 (segment (start 191.553677 127.572106) (end 192.067891 128.08632) (width 0.3) (layer "F.Cu") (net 1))
 (segment (start 192.067891 128.08632) (end 192.067891 130.072106) (width 0.3) (layer "F.Cu") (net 1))
 (segment (start 178.442893 135.107107) (end 178.442893 135.282107) (width 0.25) (layer "F.Cu") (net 1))
 (segment (start 182.767891 130.597106) (end 182.767891 131.682109) (width 0.3) (layer "F.Cu") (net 1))
 (segment (start 179.442893 134.107107) (end 178.442893 135.107107) (width 0.3) (layer "F.Cu") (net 1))
 (segment (start 182.767891 131.682109) (end 180.342893 134.107107) (width 0.3) (layer "F.Cu") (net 1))
 (segment (start 186.917891 127.572106) (end 191.553677 127.572106) (width 0.3) (layer "F.Cu") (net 1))
 (segment (start 192.210784 130.214999) (end 192.067891 130.072106) (width 0.3) (layer "F.Cu") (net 1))
 (segment (start 172.312893 115.407107) (end 173.492893 116.587107) (width 0.8) (layer "F.Cu") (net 7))
 (segment (start 173.492893 118.407107) (end 170.482893 118.407107) (width 2) (layer "F.Cu") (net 7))
 (segment (start 167.612893 115.407107) (end 172.312893 115.407107) (width 0.8) (layer "F.Cu") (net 7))
 (segment (start 173.492893 116.587107) (end 173.492893 118.407107) (width 0.8) (layer "F.Cu") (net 7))
 (segment (start 166.582893 118.487107) (end 166.582893 116.437107) (width 0.8) (layer "F.Cu") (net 7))
 (segment (start 166.582893 116.437107) (end 167.612893 115.407107) (width 0.8) (layer "F.Cu") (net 7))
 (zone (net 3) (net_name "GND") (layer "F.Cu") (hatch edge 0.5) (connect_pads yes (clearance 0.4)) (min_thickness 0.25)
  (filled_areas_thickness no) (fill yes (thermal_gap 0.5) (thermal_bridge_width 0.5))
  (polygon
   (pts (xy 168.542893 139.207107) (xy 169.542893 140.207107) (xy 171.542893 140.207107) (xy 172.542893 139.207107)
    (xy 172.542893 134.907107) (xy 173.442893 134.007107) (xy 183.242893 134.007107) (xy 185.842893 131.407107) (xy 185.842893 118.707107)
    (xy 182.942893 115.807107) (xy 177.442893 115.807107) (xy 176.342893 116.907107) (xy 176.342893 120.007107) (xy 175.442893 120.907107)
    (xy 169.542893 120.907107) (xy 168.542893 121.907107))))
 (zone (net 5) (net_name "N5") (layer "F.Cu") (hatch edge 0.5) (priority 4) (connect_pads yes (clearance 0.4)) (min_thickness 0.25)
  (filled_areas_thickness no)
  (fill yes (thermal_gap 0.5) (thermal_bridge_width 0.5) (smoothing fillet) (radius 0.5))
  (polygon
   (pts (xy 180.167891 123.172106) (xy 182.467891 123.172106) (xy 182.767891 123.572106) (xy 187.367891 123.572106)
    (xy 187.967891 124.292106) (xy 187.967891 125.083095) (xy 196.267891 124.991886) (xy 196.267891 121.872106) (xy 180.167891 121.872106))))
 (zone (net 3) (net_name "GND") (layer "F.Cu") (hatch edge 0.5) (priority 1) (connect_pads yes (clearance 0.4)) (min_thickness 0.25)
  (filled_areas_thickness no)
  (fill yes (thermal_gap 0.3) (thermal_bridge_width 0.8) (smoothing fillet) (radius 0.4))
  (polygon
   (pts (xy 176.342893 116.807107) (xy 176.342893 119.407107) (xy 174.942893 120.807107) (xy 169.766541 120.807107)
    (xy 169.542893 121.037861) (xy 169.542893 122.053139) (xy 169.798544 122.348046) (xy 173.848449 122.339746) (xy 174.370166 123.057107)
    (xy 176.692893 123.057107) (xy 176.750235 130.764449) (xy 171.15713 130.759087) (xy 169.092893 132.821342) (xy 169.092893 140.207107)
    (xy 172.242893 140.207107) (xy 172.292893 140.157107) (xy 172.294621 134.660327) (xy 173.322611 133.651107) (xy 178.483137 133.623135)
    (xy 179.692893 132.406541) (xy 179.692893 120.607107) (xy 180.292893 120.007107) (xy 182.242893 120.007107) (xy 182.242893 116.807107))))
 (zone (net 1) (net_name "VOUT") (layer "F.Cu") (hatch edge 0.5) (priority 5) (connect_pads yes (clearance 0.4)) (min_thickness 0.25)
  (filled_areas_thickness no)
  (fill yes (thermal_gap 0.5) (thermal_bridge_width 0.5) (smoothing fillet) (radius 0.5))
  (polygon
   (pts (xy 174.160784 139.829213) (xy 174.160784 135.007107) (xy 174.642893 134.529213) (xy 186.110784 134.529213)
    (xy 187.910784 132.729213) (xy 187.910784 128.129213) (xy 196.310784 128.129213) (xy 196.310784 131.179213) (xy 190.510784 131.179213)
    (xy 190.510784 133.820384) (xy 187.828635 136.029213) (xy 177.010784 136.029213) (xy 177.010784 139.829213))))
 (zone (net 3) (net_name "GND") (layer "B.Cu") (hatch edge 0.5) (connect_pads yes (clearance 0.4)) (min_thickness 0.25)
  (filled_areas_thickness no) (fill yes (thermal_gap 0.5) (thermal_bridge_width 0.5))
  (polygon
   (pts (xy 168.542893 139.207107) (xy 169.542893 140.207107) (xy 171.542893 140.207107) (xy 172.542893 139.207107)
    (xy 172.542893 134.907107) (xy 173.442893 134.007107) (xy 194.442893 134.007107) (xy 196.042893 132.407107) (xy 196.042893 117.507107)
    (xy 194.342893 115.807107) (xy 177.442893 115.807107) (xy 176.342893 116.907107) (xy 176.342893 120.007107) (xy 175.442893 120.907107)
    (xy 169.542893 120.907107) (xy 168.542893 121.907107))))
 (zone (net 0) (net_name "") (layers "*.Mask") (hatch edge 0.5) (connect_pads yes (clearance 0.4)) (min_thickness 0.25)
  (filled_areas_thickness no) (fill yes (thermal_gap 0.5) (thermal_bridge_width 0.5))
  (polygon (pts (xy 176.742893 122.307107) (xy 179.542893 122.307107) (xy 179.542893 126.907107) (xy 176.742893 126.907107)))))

